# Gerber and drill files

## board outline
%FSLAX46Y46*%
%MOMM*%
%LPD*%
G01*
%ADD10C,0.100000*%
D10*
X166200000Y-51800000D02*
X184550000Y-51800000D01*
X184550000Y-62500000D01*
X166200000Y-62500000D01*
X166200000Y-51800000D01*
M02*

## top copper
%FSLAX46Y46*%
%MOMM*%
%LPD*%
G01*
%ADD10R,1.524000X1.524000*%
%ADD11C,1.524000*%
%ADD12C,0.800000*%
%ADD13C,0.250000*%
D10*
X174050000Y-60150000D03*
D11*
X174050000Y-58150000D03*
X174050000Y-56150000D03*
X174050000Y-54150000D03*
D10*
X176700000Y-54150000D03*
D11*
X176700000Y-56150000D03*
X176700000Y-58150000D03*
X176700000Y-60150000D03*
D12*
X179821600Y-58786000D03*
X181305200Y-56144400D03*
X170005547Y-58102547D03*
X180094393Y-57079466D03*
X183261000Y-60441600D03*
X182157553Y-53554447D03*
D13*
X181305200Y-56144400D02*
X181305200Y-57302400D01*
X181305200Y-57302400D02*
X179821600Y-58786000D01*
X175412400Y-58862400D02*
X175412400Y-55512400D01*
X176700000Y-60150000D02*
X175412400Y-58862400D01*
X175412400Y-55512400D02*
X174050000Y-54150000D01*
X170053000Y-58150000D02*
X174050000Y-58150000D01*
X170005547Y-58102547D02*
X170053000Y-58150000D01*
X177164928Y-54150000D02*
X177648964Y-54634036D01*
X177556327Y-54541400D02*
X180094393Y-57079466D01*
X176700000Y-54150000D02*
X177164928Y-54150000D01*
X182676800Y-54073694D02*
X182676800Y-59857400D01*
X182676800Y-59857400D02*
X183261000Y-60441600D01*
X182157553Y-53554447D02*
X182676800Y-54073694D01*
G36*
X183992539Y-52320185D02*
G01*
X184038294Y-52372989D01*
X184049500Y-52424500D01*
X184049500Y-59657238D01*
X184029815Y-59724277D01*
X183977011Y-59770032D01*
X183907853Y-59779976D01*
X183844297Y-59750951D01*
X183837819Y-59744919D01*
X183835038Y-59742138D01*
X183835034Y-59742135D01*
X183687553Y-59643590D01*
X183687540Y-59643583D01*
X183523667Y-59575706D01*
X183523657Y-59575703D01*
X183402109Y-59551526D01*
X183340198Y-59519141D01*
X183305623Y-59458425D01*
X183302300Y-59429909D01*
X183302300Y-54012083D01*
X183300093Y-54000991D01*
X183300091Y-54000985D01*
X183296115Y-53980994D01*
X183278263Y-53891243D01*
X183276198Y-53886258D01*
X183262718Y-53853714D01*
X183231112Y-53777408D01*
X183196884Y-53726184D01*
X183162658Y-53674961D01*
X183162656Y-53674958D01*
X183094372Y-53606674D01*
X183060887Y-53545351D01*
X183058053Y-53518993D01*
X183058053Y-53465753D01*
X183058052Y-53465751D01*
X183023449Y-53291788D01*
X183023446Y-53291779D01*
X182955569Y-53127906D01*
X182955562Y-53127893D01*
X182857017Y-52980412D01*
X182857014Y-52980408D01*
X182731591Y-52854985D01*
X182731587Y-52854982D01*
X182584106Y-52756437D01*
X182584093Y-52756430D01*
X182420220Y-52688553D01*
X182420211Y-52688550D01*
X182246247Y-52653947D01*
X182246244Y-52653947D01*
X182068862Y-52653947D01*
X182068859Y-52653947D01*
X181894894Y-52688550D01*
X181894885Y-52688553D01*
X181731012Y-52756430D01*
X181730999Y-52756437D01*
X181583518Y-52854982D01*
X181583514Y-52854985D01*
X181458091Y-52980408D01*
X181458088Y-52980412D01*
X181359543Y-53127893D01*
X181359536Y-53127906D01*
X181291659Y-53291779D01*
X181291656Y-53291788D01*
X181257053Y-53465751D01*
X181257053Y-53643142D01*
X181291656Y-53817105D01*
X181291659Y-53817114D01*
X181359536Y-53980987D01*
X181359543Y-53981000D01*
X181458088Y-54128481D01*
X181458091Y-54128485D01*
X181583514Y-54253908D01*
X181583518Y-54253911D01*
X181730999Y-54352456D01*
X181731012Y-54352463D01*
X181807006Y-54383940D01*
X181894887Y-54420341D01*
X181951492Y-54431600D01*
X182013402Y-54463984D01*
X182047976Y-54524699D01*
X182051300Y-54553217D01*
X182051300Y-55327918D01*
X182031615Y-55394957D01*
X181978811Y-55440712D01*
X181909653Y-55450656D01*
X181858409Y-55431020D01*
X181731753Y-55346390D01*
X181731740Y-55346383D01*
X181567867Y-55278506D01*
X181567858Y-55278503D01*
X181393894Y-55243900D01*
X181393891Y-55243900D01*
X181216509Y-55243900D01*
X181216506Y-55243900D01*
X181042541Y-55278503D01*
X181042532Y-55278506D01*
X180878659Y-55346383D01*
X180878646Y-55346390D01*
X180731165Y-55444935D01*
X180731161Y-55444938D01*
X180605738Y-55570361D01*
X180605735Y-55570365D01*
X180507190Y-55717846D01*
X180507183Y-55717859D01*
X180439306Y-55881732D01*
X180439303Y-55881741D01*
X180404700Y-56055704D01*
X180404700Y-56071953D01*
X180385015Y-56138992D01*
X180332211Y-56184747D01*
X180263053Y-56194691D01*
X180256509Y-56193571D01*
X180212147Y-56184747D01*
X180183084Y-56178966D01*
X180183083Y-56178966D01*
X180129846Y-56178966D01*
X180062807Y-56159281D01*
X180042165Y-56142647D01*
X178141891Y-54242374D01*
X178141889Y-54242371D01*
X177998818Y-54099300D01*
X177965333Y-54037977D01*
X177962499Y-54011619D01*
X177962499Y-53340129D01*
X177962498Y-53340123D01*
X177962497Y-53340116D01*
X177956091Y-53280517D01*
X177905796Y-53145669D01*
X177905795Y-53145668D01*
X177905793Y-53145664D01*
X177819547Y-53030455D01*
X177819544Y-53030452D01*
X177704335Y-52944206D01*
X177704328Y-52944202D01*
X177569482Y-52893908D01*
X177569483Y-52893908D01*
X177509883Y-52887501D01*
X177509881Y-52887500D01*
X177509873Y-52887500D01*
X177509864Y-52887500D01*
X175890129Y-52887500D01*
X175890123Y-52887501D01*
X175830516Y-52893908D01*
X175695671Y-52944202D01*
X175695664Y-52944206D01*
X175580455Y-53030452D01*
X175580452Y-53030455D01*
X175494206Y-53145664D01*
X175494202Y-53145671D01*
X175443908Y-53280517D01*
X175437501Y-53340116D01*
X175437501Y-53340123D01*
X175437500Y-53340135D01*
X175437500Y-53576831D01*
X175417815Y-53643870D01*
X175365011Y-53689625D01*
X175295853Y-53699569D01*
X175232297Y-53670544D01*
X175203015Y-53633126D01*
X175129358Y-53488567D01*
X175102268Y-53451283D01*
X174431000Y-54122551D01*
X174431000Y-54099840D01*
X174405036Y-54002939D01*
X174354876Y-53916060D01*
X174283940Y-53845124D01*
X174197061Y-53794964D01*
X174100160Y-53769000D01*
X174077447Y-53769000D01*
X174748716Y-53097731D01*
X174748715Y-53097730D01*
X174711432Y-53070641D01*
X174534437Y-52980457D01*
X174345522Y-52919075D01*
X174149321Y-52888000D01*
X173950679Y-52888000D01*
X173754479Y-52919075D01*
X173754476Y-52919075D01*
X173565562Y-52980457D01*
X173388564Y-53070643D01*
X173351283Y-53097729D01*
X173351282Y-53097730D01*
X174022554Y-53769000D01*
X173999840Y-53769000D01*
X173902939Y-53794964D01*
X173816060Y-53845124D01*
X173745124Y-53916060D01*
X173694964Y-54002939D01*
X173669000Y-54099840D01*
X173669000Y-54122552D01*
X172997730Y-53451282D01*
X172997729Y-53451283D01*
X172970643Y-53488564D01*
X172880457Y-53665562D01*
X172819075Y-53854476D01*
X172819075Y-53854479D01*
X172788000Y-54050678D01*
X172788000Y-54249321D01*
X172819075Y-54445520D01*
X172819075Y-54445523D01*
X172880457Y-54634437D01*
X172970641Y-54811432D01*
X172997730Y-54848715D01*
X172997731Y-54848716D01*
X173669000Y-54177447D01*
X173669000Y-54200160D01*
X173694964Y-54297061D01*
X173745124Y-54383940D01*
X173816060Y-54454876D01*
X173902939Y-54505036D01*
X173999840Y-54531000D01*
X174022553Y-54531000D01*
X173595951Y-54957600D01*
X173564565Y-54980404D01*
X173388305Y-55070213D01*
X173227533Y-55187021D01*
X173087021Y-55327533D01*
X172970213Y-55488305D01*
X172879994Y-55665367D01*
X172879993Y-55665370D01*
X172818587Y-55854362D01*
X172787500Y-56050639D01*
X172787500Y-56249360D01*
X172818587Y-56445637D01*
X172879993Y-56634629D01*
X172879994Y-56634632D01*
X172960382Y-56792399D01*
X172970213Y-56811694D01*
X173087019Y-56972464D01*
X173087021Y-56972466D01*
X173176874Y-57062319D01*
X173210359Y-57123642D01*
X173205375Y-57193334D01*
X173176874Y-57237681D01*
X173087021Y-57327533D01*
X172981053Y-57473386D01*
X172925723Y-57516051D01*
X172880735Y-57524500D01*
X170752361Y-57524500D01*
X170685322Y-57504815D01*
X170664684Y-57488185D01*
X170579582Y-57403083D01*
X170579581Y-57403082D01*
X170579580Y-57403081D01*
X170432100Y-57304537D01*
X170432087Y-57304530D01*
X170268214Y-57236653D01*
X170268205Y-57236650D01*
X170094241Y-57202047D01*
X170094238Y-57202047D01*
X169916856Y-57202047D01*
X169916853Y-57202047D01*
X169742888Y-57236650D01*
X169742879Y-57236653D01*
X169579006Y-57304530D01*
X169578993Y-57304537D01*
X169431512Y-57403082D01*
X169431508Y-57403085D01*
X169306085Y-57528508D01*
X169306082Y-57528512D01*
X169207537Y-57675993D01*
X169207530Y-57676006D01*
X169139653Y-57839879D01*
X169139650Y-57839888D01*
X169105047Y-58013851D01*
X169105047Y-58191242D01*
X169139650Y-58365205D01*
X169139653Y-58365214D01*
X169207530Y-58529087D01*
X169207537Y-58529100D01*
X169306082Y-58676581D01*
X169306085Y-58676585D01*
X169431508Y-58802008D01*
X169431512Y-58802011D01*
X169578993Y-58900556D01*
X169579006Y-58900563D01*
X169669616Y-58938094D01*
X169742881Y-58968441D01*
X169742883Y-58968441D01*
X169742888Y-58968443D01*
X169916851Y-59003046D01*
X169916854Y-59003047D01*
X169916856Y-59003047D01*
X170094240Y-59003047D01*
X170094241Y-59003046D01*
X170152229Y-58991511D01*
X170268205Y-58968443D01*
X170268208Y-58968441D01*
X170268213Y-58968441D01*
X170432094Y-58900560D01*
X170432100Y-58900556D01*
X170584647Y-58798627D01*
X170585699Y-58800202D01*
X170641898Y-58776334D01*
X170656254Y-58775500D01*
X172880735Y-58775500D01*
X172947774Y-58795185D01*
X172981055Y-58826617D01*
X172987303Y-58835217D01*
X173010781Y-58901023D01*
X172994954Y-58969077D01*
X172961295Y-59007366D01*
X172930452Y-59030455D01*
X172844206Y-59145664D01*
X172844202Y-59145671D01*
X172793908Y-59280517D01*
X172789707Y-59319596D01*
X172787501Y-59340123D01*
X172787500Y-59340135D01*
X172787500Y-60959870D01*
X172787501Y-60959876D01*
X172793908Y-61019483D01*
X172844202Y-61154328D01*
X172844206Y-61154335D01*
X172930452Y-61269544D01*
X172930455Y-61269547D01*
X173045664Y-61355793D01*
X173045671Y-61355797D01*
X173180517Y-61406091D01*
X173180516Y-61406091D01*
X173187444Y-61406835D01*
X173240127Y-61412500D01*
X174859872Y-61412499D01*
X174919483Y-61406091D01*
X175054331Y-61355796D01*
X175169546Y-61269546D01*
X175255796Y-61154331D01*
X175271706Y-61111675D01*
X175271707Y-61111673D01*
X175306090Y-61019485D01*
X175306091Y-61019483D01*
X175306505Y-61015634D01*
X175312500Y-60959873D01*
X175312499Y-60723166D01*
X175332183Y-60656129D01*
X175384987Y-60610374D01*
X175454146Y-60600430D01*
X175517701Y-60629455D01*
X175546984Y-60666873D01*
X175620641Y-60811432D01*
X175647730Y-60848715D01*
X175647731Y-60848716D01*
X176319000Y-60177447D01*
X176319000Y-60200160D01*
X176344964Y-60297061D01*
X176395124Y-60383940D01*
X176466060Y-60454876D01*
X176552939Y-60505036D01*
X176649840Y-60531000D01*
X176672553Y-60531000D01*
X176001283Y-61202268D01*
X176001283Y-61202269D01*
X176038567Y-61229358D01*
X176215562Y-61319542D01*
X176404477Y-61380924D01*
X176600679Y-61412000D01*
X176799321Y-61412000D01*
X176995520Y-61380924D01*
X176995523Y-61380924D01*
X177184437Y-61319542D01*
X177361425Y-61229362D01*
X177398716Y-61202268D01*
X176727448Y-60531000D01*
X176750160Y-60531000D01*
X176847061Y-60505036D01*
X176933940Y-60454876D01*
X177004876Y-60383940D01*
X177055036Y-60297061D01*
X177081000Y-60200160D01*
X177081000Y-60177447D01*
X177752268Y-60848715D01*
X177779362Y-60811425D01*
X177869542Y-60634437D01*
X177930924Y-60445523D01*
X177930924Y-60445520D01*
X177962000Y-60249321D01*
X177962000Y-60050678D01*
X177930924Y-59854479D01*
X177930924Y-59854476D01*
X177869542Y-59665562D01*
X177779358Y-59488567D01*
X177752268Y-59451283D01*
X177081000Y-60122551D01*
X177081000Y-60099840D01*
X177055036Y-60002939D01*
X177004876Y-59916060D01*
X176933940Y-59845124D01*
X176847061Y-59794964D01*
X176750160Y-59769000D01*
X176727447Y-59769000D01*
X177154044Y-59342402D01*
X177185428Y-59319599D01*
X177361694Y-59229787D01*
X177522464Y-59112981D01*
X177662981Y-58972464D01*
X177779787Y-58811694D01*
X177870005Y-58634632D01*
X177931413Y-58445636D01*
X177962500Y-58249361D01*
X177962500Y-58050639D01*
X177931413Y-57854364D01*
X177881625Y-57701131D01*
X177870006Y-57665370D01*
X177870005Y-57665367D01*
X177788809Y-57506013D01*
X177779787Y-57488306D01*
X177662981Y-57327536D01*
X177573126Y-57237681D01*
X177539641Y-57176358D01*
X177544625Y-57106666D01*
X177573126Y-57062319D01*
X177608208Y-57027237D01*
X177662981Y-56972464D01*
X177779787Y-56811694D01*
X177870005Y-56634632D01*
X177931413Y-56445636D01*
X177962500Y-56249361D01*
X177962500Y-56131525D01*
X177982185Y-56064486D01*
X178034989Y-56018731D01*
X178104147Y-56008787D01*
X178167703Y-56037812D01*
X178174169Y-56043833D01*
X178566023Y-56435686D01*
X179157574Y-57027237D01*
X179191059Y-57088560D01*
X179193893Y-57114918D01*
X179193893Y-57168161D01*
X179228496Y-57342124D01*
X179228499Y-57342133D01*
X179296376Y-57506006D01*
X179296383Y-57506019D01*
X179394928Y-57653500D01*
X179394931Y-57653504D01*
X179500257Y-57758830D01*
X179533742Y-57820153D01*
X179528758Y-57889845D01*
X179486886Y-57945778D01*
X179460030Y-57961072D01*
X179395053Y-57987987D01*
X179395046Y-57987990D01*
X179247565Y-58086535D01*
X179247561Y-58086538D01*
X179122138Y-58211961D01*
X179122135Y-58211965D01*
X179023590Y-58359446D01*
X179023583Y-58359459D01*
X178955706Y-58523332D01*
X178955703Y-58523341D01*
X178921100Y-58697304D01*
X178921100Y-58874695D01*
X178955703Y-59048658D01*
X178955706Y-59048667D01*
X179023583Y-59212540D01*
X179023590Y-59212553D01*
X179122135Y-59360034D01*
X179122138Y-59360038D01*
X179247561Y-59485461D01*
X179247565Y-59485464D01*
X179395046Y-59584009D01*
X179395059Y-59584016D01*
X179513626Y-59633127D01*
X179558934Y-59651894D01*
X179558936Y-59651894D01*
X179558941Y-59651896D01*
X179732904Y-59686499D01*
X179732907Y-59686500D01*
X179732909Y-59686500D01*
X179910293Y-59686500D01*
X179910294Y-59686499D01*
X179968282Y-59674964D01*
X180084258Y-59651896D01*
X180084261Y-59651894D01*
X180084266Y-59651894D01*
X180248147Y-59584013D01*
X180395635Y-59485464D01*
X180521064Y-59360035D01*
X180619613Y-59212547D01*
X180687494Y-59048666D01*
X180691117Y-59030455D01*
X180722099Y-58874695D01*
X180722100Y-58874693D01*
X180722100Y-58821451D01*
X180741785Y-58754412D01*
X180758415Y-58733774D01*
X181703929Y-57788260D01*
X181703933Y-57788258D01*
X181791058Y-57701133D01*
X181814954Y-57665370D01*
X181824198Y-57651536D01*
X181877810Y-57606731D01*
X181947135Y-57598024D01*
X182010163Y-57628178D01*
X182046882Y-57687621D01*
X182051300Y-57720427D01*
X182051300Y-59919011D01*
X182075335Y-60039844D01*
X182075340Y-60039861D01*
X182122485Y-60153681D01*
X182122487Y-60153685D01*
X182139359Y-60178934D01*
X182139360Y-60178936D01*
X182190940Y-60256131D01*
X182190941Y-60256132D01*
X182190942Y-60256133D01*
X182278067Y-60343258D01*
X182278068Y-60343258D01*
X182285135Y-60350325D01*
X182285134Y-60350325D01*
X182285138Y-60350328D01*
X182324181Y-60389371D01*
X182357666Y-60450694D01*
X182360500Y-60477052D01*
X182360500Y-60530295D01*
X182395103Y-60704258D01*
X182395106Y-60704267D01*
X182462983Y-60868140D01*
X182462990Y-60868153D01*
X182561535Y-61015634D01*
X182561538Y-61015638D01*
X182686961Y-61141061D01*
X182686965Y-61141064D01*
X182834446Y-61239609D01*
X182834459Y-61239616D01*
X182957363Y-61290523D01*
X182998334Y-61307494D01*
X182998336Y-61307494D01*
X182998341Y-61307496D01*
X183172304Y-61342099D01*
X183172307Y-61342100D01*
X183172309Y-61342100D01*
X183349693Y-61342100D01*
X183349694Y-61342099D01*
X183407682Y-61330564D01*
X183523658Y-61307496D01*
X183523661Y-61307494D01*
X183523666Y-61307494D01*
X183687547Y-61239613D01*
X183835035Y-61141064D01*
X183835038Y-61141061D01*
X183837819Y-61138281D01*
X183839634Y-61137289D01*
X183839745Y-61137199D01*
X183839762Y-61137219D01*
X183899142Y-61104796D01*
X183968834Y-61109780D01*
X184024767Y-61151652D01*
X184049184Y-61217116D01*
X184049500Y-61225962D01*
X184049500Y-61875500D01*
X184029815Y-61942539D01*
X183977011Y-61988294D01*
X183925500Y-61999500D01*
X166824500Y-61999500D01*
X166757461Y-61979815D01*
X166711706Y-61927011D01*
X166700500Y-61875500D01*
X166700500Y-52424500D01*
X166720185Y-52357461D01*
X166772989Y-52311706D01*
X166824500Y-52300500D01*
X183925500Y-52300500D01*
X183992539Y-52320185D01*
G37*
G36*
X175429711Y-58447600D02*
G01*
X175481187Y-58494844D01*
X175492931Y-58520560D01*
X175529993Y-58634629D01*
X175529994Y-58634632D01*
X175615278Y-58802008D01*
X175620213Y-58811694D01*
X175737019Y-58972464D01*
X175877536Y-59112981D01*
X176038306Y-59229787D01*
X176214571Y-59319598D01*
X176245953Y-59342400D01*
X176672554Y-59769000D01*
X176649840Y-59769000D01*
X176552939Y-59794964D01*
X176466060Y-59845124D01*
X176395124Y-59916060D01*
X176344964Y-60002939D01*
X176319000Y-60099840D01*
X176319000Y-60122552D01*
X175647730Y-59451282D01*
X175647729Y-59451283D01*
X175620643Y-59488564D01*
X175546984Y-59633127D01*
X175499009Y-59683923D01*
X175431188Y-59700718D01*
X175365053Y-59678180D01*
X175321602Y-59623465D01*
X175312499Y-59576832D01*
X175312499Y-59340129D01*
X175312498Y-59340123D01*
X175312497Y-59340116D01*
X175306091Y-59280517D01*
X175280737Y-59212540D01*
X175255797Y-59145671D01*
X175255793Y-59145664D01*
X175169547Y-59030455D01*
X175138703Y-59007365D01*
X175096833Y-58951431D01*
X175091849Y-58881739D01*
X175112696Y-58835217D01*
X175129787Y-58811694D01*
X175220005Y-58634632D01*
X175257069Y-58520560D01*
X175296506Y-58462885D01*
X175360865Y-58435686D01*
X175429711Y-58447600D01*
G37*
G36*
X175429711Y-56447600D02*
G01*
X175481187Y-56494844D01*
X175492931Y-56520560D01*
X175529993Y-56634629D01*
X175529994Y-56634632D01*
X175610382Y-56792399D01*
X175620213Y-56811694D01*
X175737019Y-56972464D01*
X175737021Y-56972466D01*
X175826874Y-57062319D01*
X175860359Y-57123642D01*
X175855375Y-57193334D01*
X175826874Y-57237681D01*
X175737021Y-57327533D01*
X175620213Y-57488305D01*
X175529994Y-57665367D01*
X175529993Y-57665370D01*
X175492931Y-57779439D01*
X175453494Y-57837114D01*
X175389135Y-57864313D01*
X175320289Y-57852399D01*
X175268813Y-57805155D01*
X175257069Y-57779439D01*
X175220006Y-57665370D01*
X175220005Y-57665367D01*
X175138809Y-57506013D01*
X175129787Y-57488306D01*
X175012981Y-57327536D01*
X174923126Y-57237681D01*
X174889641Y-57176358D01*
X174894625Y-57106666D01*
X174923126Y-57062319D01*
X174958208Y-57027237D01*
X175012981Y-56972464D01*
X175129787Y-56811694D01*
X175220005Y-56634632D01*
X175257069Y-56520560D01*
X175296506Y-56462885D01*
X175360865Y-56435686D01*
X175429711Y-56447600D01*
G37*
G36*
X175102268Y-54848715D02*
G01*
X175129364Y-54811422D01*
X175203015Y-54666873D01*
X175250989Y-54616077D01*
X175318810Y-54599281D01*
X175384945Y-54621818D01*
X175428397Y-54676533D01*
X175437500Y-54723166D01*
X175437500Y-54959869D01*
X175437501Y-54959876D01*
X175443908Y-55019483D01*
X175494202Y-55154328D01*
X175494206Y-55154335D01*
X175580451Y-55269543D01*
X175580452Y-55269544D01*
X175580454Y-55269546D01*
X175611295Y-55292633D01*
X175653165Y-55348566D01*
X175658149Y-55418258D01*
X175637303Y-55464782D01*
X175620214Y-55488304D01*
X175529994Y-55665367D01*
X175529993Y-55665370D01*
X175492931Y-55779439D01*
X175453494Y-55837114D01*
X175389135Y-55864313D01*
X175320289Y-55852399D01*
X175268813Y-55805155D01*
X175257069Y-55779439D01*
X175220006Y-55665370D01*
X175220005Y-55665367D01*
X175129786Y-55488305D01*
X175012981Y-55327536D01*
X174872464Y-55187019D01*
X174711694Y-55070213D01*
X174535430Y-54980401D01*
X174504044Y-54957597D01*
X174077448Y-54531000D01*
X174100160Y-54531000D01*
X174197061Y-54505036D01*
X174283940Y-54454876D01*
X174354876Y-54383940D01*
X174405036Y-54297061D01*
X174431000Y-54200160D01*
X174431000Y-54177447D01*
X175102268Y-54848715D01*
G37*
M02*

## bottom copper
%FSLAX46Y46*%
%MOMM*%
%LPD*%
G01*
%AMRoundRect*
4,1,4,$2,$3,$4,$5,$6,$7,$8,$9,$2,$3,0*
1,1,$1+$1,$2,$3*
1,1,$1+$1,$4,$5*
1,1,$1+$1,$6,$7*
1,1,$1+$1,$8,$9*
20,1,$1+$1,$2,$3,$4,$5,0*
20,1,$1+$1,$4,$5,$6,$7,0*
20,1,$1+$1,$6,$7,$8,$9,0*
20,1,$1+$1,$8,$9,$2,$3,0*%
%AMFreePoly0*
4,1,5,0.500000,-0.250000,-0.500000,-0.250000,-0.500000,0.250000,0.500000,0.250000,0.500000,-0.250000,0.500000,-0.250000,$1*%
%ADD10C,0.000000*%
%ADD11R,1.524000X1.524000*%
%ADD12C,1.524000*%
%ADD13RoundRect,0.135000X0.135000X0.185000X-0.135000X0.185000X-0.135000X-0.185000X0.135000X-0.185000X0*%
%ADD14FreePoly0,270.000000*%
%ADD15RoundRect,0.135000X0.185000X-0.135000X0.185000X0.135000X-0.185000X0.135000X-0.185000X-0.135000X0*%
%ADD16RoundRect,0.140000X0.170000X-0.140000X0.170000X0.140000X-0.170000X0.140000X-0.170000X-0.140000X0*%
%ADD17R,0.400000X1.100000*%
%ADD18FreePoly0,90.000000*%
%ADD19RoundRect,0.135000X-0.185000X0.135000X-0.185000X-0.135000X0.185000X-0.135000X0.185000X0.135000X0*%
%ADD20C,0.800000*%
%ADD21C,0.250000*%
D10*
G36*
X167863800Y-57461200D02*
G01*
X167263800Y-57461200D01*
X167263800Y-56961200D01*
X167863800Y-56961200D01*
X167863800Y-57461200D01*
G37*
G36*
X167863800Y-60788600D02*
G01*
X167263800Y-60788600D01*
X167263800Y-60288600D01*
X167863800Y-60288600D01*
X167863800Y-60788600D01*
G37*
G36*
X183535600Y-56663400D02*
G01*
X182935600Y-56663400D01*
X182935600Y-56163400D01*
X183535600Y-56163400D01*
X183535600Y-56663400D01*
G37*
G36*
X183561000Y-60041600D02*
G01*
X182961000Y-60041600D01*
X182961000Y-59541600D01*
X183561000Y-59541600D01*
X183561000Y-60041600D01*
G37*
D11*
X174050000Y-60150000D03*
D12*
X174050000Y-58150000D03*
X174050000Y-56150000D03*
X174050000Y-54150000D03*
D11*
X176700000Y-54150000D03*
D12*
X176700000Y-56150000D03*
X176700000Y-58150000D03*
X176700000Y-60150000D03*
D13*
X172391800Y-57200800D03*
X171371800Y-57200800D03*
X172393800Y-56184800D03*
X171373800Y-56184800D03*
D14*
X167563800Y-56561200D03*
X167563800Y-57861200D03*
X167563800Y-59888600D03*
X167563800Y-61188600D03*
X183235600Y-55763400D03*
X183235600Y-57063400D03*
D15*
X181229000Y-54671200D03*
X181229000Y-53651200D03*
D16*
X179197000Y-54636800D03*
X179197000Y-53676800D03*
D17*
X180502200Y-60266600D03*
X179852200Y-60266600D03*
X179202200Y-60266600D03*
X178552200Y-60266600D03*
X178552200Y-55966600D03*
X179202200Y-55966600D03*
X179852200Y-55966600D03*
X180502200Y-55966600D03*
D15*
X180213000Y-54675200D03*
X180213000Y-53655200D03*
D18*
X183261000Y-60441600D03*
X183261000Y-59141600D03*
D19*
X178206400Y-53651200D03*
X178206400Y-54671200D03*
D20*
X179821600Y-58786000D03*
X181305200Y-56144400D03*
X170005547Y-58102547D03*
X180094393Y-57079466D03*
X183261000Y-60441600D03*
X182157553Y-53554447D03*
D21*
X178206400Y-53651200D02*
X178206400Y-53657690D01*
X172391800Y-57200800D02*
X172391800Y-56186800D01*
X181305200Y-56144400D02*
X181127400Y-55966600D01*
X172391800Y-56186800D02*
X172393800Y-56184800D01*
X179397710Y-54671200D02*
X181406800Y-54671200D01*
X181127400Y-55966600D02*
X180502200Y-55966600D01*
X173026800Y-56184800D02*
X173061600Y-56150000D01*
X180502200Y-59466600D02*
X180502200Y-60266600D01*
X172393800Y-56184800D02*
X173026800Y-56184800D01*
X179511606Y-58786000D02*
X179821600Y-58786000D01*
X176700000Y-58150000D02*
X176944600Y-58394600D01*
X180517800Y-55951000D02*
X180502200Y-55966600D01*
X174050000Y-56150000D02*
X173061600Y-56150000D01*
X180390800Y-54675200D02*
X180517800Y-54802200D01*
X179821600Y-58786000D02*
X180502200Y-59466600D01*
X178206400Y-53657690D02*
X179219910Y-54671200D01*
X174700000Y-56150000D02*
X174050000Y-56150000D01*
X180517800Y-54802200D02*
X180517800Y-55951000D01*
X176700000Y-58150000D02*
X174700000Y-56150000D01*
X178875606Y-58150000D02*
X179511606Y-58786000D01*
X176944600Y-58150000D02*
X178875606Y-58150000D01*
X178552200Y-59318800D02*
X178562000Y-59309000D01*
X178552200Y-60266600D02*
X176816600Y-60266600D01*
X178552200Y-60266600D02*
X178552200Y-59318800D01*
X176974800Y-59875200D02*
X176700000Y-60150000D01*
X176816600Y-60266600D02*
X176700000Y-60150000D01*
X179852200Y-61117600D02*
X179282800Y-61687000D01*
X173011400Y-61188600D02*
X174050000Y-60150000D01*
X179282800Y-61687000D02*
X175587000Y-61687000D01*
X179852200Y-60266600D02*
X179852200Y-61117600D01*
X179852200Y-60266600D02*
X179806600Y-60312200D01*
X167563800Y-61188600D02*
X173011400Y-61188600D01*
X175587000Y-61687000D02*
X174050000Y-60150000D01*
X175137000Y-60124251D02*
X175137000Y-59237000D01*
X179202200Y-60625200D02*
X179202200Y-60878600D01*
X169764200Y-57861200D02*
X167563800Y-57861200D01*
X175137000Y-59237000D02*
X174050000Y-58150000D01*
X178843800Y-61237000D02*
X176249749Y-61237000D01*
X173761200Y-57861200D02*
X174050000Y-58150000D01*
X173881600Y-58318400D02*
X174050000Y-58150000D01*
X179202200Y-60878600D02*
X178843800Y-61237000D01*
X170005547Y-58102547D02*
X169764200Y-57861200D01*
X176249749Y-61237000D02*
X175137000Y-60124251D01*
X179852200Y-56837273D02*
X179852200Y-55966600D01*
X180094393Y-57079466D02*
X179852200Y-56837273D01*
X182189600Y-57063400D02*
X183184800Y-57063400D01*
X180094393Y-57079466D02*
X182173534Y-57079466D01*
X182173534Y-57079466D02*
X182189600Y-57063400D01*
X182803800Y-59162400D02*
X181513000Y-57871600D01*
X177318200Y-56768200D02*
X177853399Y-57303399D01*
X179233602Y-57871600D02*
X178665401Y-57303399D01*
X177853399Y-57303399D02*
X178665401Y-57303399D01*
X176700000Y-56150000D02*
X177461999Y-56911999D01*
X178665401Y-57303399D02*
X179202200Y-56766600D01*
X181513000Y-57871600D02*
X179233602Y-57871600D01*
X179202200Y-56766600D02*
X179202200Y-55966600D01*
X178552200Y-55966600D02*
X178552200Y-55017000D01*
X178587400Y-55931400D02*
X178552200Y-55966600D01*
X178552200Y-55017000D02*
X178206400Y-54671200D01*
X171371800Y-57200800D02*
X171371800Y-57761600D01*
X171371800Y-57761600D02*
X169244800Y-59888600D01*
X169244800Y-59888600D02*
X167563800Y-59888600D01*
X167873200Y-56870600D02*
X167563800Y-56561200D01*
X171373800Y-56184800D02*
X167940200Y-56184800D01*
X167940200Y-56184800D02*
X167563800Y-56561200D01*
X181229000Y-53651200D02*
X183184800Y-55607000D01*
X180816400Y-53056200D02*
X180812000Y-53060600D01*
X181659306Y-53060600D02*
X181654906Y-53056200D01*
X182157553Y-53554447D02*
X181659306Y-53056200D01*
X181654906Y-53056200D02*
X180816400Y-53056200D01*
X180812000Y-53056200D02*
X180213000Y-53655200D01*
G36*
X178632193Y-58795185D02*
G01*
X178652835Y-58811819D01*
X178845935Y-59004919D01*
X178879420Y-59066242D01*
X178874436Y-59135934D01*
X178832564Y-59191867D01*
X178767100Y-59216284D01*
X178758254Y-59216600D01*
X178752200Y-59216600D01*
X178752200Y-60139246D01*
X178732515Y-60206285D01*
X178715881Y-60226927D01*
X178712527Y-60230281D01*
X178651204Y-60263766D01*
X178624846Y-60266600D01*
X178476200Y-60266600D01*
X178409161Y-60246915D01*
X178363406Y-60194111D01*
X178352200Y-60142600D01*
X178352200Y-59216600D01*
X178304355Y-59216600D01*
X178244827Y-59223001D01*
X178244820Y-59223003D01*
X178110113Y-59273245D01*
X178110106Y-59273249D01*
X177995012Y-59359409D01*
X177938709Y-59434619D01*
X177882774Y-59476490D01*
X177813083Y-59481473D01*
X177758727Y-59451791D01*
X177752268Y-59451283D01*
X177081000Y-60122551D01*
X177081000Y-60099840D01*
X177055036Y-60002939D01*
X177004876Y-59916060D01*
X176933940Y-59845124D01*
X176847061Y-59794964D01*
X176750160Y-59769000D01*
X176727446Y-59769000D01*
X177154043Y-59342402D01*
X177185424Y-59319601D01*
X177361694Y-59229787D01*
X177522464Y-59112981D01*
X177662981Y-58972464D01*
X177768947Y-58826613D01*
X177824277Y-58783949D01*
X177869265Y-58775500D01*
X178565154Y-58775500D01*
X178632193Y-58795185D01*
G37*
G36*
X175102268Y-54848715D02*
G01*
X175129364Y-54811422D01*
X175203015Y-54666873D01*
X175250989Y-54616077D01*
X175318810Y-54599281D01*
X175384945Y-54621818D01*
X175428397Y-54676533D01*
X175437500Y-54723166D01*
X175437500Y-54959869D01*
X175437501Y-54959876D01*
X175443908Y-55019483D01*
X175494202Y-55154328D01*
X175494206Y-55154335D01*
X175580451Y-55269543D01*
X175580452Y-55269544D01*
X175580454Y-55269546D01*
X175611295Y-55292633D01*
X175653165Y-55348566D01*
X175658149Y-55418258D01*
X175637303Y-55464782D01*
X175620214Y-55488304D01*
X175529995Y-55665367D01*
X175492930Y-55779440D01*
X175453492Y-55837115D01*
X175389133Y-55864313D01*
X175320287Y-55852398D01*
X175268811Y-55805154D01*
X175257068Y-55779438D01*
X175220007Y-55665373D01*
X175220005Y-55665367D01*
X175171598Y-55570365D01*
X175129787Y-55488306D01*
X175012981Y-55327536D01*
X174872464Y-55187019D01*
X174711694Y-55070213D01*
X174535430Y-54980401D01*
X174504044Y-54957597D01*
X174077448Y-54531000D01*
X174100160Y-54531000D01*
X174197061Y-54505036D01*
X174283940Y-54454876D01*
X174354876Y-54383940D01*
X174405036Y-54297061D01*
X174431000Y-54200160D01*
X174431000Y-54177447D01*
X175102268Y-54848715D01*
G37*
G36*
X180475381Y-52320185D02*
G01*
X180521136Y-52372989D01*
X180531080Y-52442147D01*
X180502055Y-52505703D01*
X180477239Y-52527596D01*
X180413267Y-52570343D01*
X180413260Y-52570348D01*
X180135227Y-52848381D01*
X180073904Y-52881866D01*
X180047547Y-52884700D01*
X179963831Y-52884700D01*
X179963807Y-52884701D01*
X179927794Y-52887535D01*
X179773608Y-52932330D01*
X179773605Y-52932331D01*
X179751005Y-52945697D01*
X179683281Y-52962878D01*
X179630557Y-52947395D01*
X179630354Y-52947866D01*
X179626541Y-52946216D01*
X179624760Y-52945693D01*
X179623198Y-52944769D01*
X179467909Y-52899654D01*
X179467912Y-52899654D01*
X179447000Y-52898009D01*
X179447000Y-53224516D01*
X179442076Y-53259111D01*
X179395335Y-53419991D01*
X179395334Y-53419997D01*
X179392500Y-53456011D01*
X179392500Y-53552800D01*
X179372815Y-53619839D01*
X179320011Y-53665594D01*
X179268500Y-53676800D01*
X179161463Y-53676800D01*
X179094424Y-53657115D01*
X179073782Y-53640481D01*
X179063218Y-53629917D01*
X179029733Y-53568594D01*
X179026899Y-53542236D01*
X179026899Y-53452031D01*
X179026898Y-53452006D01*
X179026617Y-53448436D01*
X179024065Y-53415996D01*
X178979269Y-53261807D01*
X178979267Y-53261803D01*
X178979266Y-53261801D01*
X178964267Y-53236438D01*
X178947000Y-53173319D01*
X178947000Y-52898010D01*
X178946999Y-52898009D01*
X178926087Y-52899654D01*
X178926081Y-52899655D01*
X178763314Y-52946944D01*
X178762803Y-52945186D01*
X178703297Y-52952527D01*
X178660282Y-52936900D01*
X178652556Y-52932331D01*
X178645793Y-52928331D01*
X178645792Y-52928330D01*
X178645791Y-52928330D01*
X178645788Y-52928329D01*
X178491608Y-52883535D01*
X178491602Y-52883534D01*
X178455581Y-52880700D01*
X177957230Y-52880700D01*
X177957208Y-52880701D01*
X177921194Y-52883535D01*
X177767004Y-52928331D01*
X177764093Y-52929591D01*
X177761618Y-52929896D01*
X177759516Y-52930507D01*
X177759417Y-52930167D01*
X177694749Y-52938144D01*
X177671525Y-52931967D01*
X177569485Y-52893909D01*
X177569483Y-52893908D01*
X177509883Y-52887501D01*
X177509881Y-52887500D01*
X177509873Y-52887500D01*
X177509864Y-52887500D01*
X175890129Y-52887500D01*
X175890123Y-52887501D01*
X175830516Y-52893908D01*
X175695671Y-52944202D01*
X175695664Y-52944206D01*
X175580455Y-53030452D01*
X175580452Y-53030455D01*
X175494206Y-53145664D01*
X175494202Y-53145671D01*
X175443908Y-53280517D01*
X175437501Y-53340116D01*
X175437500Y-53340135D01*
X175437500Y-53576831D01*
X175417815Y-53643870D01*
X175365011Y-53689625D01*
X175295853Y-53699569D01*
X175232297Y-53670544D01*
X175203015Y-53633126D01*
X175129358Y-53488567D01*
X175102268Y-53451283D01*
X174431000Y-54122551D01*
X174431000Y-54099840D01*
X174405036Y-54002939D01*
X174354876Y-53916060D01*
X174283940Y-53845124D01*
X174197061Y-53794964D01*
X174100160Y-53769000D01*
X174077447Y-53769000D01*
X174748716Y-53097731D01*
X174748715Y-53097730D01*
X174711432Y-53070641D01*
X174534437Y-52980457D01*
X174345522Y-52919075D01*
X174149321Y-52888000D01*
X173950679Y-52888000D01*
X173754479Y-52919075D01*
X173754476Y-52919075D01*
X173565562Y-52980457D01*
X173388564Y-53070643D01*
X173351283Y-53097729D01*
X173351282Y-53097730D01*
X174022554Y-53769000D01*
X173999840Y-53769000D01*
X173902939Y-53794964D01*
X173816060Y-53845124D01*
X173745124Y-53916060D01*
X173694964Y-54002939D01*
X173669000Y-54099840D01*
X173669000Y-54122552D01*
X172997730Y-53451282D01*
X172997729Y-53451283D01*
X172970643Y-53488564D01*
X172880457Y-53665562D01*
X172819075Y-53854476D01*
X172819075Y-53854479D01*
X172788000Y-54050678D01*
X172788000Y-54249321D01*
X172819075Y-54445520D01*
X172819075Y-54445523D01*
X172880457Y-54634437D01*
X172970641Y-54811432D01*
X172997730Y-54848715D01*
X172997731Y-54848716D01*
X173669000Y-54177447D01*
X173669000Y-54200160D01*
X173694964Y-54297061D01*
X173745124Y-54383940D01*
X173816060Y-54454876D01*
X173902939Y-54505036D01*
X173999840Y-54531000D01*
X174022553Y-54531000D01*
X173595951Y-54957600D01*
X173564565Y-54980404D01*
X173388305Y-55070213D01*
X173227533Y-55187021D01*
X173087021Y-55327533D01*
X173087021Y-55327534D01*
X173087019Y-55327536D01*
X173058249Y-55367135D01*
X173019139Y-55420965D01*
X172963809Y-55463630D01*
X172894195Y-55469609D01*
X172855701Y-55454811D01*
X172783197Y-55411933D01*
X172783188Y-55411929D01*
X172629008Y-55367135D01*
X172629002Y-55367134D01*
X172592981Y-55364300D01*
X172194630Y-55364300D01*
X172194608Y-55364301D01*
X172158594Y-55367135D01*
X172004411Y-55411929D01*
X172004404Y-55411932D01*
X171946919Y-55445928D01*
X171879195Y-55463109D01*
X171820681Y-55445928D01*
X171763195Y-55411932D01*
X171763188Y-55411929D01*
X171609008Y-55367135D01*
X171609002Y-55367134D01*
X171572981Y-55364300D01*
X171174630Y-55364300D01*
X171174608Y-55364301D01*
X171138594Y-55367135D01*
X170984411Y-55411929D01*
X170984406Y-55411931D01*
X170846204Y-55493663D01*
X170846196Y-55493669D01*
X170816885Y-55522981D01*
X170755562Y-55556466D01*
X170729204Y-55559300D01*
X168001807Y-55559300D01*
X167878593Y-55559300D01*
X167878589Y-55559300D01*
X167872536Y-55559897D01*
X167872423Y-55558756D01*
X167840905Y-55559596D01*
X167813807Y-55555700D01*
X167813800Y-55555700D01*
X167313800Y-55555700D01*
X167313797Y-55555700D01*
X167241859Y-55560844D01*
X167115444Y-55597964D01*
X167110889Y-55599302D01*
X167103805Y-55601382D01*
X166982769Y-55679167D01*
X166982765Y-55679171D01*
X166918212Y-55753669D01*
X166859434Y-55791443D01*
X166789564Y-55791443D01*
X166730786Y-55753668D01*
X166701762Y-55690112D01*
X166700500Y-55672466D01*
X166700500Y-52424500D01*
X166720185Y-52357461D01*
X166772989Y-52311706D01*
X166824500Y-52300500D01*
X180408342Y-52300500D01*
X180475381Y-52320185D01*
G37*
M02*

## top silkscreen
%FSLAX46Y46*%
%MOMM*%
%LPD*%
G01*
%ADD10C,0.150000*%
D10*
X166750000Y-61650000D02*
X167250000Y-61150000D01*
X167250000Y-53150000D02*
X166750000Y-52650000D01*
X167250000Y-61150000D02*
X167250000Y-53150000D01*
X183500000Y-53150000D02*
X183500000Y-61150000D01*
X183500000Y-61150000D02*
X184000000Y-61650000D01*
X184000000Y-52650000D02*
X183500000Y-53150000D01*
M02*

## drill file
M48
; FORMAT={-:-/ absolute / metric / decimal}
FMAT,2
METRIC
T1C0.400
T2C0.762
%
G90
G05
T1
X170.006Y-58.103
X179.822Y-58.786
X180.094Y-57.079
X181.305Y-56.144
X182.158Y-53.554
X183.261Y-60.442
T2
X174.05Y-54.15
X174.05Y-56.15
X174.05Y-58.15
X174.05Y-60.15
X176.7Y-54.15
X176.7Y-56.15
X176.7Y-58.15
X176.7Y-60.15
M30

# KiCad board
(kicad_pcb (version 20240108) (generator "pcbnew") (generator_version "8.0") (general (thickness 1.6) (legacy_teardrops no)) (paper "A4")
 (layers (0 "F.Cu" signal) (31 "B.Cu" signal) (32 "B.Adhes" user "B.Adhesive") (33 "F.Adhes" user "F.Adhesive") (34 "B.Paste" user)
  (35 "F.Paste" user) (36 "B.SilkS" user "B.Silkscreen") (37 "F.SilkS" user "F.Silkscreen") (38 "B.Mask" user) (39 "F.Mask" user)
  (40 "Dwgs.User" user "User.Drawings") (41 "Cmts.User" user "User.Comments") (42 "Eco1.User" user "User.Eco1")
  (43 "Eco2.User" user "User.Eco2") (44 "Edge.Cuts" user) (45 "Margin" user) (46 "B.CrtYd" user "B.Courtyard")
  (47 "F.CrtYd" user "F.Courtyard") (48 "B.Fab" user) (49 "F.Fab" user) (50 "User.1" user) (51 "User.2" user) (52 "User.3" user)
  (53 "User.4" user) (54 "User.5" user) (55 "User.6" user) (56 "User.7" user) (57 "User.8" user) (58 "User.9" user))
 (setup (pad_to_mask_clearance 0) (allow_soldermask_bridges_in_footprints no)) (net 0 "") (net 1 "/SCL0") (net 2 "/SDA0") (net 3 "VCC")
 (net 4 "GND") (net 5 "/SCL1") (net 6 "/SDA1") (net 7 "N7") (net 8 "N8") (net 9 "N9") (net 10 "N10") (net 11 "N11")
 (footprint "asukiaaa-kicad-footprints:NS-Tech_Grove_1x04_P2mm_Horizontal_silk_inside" (layer "F.Cu") (at 174.05 57.15 180)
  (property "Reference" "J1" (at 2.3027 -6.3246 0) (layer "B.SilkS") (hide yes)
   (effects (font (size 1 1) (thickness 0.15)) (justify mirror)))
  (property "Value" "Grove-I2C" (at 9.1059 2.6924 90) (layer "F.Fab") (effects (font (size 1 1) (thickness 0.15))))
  (fp_line (start 7.3 -4.5) (end 6.8 -4) (stroke (width 0.15) (type solid)) (layer "F.SilkS"))
  (fp_line (start 6.8 4) (end 7.3 4.5) (stroke (width 0.15) (type solid)) (layer "F.SilkS"))
  (fp_line (start 6.8 -4) (end 6.8 4) (stroke (width 0.15) (type solid)) (layer "F.SilkS"))
  (pad "1" thru_hole rect (at 0 -3 180) (size 1.524 1.524) (drill 0.762) (layers "*.Cu" "*.Mask") (remove_unused_layers no) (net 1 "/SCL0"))
  (pad "2" thru_hole circle (at 0 -1 180) (size 1.524 1.524) (drill 0.762) (layers "*.Cu" "*.Mask") (remove_unused_layers no)
   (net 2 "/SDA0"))
  (pad "3" thru_hole circle (at 0 1 180) (size 1.524 1.524) (drill 0.762) (layers "*.Cu" "*.Mask") (remove_unused_layers no) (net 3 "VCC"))
  (pad "4" thru_hole circle (at 0 3 180) (size 1.524 1.524) (drill 0.762) (layers "*.Cu" "*.Mask") (remove_unused_layers no) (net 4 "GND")))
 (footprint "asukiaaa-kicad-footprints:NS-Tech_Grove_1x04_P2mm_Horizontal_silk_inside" (layer "F.Cu") (at 176.7 57.15)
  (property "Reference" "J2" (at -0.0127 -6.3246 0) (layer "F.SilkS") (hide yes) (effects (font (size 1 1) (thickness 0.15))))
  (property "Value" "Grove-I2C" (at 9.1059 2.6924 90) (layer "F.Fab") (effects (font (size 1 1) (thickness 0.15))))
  (fp_line (start 6.8 -4) (end 6.8 4) (stroke (width 0.15) (type solid)) (layer "F.SilkS"))
  (fp_line (start 6.8 4) (end 7.3 4.5) (stroke (width 0.15) (type solid)) (layer "F.SilkS"))
  (fp_line (start 7.3 -4.5) (end 6.8 -4) (stroke (width 0.15) (type solid)) (layer "F.SilkS"))
  (pad "1" thru_hole rect (at 0 -3) (size 1.524 1.524) (drill 0.762) (layers "*.Cu" "*.Mask") (remove_unused_layers no) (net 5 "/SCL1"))
  (pad "2" thru_hole circle (at 0 -1) (size 1.524 1.524) (drill 0.762) (layers "*.Cu" "*.Mask") (remove_unused_layers no) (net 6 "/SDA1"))
  (pad "3" thru_hole circle (at 0 1) (size 1.524 1.524) (drill 0.762) (layers "*.Cu" "*.Mask") (remove_unused_layers no) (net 3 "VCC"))
  (pad "4" thru_hole circle (at 0 3) (size 1.524 1.524) (drill 0.762) (layers "*.Cu" "*.Mask") (remove_unused_layers no) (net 4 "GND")))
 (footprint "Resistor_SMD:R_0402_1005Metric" (layer "B.Cu") (at 171.8818 57.2008 180)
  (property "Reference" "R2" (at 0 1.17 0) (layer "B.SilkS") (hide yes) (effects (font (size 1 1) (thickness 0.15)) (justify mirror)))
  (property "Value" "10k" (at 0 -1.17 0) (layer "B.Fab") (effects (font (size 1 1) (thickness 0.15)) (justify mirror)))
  (pad "1" smd roundrect (at -0.51 0 180) (size 0.54 0.64) (layers "B.Cu" "B.Paste" "B.Mask") (roundrect_rratio 0.25) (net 3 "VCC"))
  (pad "2" smd roundrect (at 0.51 0 180) (size 0.54 0.64) (layers "B.Cu" "B.Paste" "B.Mask") (roundrect_rratio 0.25) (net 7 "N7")))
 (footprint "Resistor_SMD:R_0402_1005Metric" (layer "B.Cu") (at 171.8838 56.1848 180)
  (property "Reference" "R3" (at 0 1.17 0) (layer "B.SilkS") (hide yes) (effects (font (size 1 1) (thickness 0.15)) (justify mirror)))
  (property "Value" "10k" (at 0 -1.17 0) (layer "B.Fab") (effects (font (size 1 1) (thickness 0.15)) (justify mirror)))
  (pad "1" smd roundrect (at -0.51 0 180) (size 0.54 0.64) (layers "B.Cu" "B.Paste" "B.Mask") (roundrect_rratio 0.25) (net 3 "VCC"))
  (pad "2" smd roundrect (at 0.51 0 180) (size 0.54 0.64) (layers "B.Cu" "B.Paste" "B.Mask") (roundrect_rratio 0.25) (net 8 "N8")))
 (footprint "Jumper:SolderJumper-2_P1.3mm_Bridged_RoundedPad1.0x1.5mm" (layer "B.Cu") (at 167.5638 57.2112 -90)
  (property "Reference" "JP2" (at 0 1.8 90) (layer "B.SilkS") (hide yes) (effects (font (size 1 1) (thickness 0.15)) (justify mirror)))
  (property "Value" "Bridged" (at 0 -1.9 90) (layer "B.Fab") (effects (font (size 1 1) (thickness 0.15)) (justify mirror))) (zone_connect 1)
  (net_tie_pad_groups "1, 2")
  (fp_poly (pts (xy 0.25 0.3) (xy -0.25 0.3) (xy -0.25 -0.3) (xy 0.25 -0.3)) (stroke (width 0) (type solid)) (fill solid) (layer "B.Cu"))
  (pad "1" smd custom (at -0.65 0 270) (size 1 0.5) (layers "B.Cu" "B.Mask") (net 8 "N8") (zone_connect 2) (thermal_bridge_angle 45)
   (options (clearance outline) (anchor rect)) (primitives))
  (pad "2" smd custom (at 0.65 0 270) (size 1 0.5) (layers "B.Cu" "B.Mask") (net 2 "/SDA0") (zone_connect 2) (thermal_bridge_angle 45)
   (options (clearance outline) (anchor rect)) (primitives)))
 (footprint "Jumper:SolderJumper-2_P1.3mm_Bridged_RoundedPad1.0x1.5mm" (layer "B.Cu") (at 167.5638 60.5386 -90)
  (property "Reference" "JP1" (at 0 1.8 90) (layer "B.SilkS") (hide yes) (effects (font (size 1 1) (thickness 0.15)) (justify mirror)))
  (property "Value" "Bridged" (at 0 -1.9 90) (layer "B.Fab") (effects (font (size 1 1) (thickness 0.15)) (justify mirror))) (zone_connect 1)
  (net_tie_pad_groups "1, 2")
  (fp_poly (pts (xy 0.25 0.3) (xy -0.25 0.3) (xy -0.25 -0.3) (xy 0.25 -0.3)) (stroke (width 0) (type solid)) (fill solid) (layer "B.Cu"))
  (pad "1" smd custom (at -0.65 0 270) (size 1 0.5) (layers "B.Cu" "B.Mask") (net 7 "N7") (zone_connect 2) (thermal_bridge_angle 45)
   (options (clearance outline) (anchor rect)) (primitives))
  (pad "2" smd custom (at 0.65 0 270) (size 1 0.5) (layers "B.Cu" "B.Mask") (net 1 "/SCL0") (zone_connect 2) (thermal_bridge_angle 45)
   (options (clearance outline) (anchor rect)) (primitives)))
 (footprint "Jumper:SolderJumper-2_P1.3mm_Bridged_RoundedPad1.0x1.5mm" (layer "B.Cu") (at 183.2356 56.4134 -90)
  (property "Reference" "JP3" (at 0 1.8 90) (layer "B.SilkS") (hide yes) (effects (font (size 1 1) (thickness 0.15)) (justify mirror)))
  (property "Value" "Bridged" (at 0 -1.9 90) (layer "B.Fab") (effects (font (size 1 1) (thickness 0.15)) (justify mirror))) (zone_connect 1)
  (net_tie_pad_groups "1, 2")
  (fp_poly (pts (xy 0.25 0.3) (xy -0.25 0.3) (xy -0.25 -0.3) (xy 0.25 -0.3)) (stroke (width 0) (type solid)) (fill solid) (layer "B.Cu"))
  (pad "1" smd custom (at -0.65 0 270) (size 1 0.5) (layers "B.Cu" "B.Mask") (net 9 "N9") (zone_connect 2) (thermal_bridge_angle 45)
   (options (clearance outline) (anchor rect)) (primitives))
  (pad "2" smd custom (at 0.65 0 270) (size 1 0.5) (layers "B.Cu" "B.Mask") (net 5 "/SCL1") (zone_connect 2) (thermal_bridge_angle 45)
   (options (clearance outline) (anchor rect)) (primitives)))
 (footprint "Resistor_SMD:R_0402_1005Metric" (layer "B.Cu") (at 181.229 54.1612 90)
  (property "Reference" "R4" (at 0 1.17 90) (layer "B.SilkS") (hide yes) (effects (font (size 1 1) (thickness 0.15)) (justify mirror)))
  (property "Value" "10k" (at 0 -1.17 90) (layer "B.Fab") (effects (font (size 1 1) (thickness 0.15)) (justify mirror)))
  (pad "1" smd roundrect (at -0.51 0 90) (size 0.54 0.64) (layers "B.Cu" "B.Paste" "B.Mask") (roundrect_rratio 0.25) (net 3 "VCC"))
  (pad "2" smd roundrect (at 0.51 0 90) (size 0.54 0.64) (layers "B.Cu" "B.Paste" "B.Mask") (roundrect_rratio 0.25) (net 9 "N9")))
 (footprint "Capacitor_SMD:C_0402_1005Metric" (layer "B.Cu") (at 179.197 54.1568 90)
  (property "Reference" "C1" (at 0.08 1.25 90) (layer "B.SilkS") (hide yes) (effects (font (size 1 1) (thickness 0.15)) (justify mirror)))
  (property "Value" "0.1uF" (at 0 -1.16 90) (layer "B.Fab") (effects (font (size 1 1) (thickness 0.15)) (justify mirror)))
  (pad "1" smd roundrect (at -0.48 0 90) (size 0.56 0.62) (layers "B.Cu" "B.Paste" "B.Mask") (roundrect_rratio 0.25) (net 3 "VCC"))
  (pad "2" smd roundrect (at 0.48 0 90) (size 0.56 0.62) (layers "B.Cu" "B.Paste" "B.Mask") (roundrect_rratio 0.25) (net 4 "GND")))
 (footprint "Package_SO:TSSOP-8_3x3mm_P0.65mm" (layer "B.Cu") (at 179.5272 58.1166 90)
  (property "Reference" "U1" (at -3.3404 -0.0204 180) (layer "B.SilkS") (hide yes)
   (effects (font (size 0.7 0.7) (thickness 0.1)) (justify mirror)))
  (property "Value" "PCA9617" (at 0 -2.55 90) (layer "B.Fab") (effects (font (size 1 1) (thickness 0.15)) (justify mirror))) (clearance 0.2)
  (pad "1" smd rect (at -2.15 0.975 90) (size 1.1 0.4) (layers "B.Cu" "B.Paste" "B.Mask") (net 3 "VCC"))
  (pad "2" smd rect (at -2.15 0.325 90) (size 1.1 0.4) (layers "B.Cu" "B.Paste" "B.Mask") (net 1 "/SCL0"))
  (pad "3" smd rect (at -2.15 -0.325 90) (size 1.1 0.4) (layers "B.Cu" "B.Paste" "B.Mask") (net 2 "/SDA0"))
  (pad "4" smd rect (at -2.15 -0.975 90) (size 1.1 0.4) (layers "B.Cu" "B.Paste" "B.Mask") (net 4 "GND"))
  (pad "5" smd rect (at 2.15 -0.975 90) (size 1.1 0.4) (layers "B.Cu" "B.Paste" "B.Mask") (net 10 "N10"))
  (pad "6" smd rect (at 2.15 -0.325 90) (size 1.1 0.4) (layers "B.Cu" "B.Paste" "B.Mask") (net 6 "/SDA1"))
  (pad "7" smd rect (at 2.15 0.325 90) (size 1.1 0.4) (layers "B.Cu" "B.Paste" "B.Mask") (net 5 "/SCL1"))
  (pad "8" smd rect (at 2.15 0.975 90) (size 1.1 0.4) (layers "B.Cu" "B.Paste" "B.Mask") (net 3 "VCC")))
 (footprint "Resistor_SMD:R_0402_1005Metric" (layer "B.Cu") (at 180.213 54.1652 90)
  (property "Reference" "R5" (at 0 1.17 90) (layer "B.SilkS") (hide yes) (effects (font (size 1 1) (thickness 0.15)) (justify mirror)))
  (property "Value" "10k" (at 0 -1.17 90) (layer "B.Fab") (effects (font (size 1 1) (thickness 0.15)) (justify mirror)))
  (pad "1" smd roundrect (at -0.51 0 90) (size 0.54 0.64) (layers "B.Cu" "B.Paste" "B.Mask") (roundrect_rratio 0.25) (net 3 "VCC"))
  (pad "2" smd roundrect (at 0.51 0 90) (size 0.54 0.64) (layers "B.Cu" "B.Paste" "B.Mask") (roundrect_rratio 0.25) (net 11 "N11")))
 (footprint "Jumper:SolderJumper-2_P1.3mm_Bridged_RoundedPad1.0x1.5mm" (layer "B.Cu") (at 183.261 59.7916 90)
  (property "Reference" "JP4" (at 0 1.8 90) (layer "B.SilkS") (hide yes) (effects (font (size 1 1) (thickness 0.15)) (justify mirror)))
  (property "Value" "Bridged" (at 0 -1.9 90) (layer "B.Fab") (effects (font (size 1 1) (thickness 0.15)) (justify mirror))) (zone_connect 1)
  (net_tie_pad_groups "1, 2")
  (fp_poly (pts (xy 0.25 0.3) (xy -0.25 0.3) (xy -0.25 -0.3) (xy 0.25 -0.3)) (stroke (width 0) (type solid)) (fill solid) (layer "B.Cu"))
  (pad "1" smd custom (at -0.65 0 90) (size 1 0.5) (layers "B.Cu" "B.Mask") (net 11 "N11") (zone_connect 2) (thermal_bridge_angle 45)
   (options (clearance outline) (anchor rect)) (primitives))
  (pad "2" smd custom (at 0.65 0 90) (size 1 0.5) (layers "B.Cu" "B.Mask") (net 6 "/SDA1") (zone_connect 2) (thermal_bridge_angle 45)
   (options (clearance outline) (anchor rect)) (primitives)))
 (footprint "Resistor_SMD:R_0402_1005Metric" (layer "B.Cu") (at 178.2064 54.1612 -90)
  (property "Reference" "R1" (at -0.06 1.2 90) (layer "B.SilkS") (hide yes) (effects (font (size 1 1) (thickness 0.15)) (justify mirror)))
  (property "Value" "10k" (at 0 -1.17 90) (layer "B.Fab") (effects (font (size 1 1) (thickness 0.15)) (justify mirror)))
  (pad "1" smd roundrect (at -0.51 0 270) (size 0.54 0.64) (layers "B.Cu" "B.Paste" "B.Mask") (roundrect_rratio 0.25) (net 3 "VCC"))
  (pad "2" smd roundrect (at 0.51 0 270) (size 0.54 0.64) (layers "B.Cu" "B.Paste" "B.Mask") (roundrect_rratio 0.25) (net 10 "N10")))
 (gr_rect (start 166.2 51.8) (end 184.55 62.5) (stroke (width 0.1) (type default)) (fill none) (layer "Edge.Cuts"))
 (segment (start 181.3052 56.1444) (end 181.3052 57.3024) (width 0.25) (layer "F.Cu") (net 3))
 (segment (start 181.3052 57.3024) (end 179.8216 58.786) (width 0.25) (layer "F.Cu") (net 3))
 (via (at 179.8216 58.786) (size 0.8) (drill 0.4) (layers "F.Cu" "B.Cu") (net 3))
 (via (at 181.3052 56.1444) (size 0.8) (drill 0.4) (layers "F.Cu" "B.Cu") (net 3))
 (segment (start 178.2064 53.6512) (end 178.2064 53.65769) (width 0.25) (layer "B.Cu") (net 3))
 (segment (start 172.3918 57.2008) (end 172.3918 56.1868) (width 0.25) (layer "B.Cu") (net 3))
 (segment (start 181.3052 56.1444) (end 181.1274 55.9666) (width 0.25) (layer "B.Cu") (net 3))
 (segment (start 172.3918 56.1868) (end 172.3938 56.1848) (width 0.25) (layer "B.Cu") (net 3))
 (segment (start 179.39771 54.6712) (end 181.4068 54.6712) (width 0.25) (layer "B.Cu") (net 3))
 (segment (start 181.1274 55.9666) (end 180.5022 55.9666) (width 0.25) (layer "B.Cu") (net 3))
 (segment (start 173.0268 56.1848) (end 173.0616 56.15) (width 0.25) (layer "B.Cu") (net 3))
 (segment (start 180.5022 59.4666) (end 180.5022 60.2666) (width 0.25) (layer "B.Cu") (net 3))
 (segment (start 172.3938 56.1848) (end 173.0268 56.1848) (width 0.25) (layer "B.Cu") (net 3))
 (segment (start 179.511606 58.786) (end 179.8216 58.786) (width 0.25) (layer "B.Cu") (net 3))
 (segment (start 176.7 58.15) (end 176.9446 58.3946) (width 0.25) (layer "B.Cu") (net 3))
 (segment (start 180.5178 55.951) (end 180.5022 55.9666) (width 0.25) (layer "B.Cu") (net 3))
 (segment (start 174.05 56.15) (end 173.0616 56.15) (width 0.25) (layer "B.Cu") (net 3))
 (segment (start 180.3908 54.6752) (end 180.5178 54.8022) (width 0.25) (layer "B.Cu") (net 3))
 (segment (start 179.8216 58.786) (end 180.5022 59.4666) (width 0.25) (layer "B.Cu") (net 3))
 (segment (start 178.2064 53.65769) (end 179.21991 54.6712) (width 0.25) (layer "B.Cu") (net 3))
 (segment (start 174.7 56.15) (end 174.05 56.15) (width 0.25) (layer "B.Cu") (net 3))
 (segment (start 180.5178 54.8022) (end 180.5178 55.951) (width 0.25) (layer "B.Cu") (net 3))
 (segment (start 176.7 58.15) (end 174.7 56.15) (width 0.25) (layer "B.Cu") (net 3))
 (segment (start 178.875606 58.15) (end 179.511606 58.786) (width 0.25) (layer "B.Cu") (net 3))
 (segment (start 176.9446 58.15) (end 178.875606 58.15) (width 0.25) (layer "B.Cu") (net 3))
 (segment (start 175.4124 58.8624) (end 175.4124 55.5124) (width 0.25) (layer "F.Cu") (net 4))
 (segment (start 176.7 60.15) (end 175.4124 58.8624) (width 0.25) (layer "F.Cu") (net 4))
 (segment (start 175.4124 55.5124) (end 174.05 54.15) (width 0.25) (layer "F.Cu") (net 4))
 (segment (start 178.5522 59.3188) (end 178.562 59.309) (width 0.25) (layer "B.Cu") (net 4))
 (segment (start 178.5522 60.2666) (end 176.8166 60.2666) (width 0.25) (layer "B.Cu") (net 4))
 (segment (start 178.5522 60.2666) (end 178.5522 59.3188) (width 0.25) (layer "B.Cu") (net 4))
 (segment (start 176.9748 59.8752) (end 176.7 60.15) (width 0.25) (layer "B.Cu") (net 4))
 (segment (start 176.8166 60.2666) (end 176.7 60.15) (width 0.25) (layer "B.Cu") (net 4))
 (segment (start 179.8522 61.1176) (end 179.2828 61.687) (width 0.25) (layer "B.Cu") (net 1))
 (segment (start 173.0114 61.1886) (end 174.05 60.15) (width 0.25) (layer "B.Cu") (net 1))
 (segment (start 179.2828 61.687) (end 175.587 61.687) (width 0.25) (layer "B.Cu") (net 1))
 (segment (start 179.8522 60.2666) (end 179.8522 61.1176) (width 0.25) (layer "B.Cu") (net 1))
 (segment (start 179.8522 60.2666) (end 179.8066 60.3122) (width 0.25) (layer "B.Cu") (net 1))
 (segment (start 167.5638 61.1886) (end 173.0114 61.1886) (width 0.25) (layer "B.Cu") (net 1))
 (segment (start 175.587 61.687) (end 174.05 60.15) (width 0.25) (layer "B.Cu") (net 1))
 (segment (start 170.053 58.15) (end 174.05 58.15) (width 0.25) (layer "F.Cu") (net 2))
 (segment (start 170.005547 58.102547) (end 170.053 58.15) (width 0.25) (layer "F.Cu") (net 2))
 (via (at 170.005547 58.102547) (size 0.8) (drill 0.4) (layers "F.Cu" "B.Cu") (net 2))
 (segment (start 175.137 60.124251) (end 175.137 59.237) (width 0.25) (layer "B.Cu") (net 2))
 (segment (start 179.2022 60.6252) (end 179.2022 60.8786) (width 0.25) (layer "B.Cu") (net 2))
 (segment (start 169.7642 57.8612) (end 167.5638 57.8612) (width 0.25) (layer "B.Cu") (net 2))
 (segment (start 175.137 59.237) (end 174.05 58.15) (width 0.25) (layer "B.Cu") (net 2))
 (segment (start 178.8438 61.237) (end 176.249749 61.237) (width 0.25) (layer "B.Cu") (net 2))
 (segment (start 173.7612 57.8612) (end 174.05 58.15) (width 0.25) (layer "B.Cu") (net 2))
 (segment (start 173.8816 58.3184) (end 174.05 58.15) (width 0.25) (layer "B.Cu") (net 2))
 (segment (start 179.2022 60.8786) (end 178.8438 61.237) (width 0.25) (layer "B.Cu") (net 2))
 (segment (start 170.005547 58.102547) (end 169.7642 57.8612) (width 0.25) (layer "B.Cu") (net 2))
 (segment (start 176.249749 61.237) (end 175.137 60.124251) (width 0.25) (layer "B.Cu") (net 2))
 (segment (start 177.164928 54.15) (end 177.648964 54.634036) (width 0.25) (layer "F.Cu") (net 5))
 (segment (start 177.556327 54.5414) (end 180.094393 57.079466) (width 0.25) (layer "F.Cu") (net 5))
 (segment (start 176.7 54.15) (end 177.164928 54.15) (width 0.25) (layer "F.Cu") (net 5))
 (via (at 180.094393 57.079466) (size 0.8) (drill 0.4) (layers "F.Cu" "B.Cu") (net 5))
 (segment (start 179.8522 56.837273) (end 179.8522 55.9666) (width 0.25) (layer "B.Cu") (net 5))
 (segment (start 180.094393 57.079466) (end 179.8522 56.837273) (width 0.25) (layer "B.Cu") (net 5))
 (segment (start 182.1896 57.0634) (end 183.1848 57.0634) (width 0.25) (layer "B.Cu") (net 5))
 (segment (start 180.094393 57.079466) (end 182.173534 57.079466) (width 0.25) (layer "B.Cu") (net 5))
 (segment (start 182.173534 57.079466) (end 182.1896 57.0634) (width 0.25) (layer "B.Cu") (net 5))
 (segment (start 182.8038 59.1624) (end 181.513 57.8716) (width 0.25) (layer "B.Cu") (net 6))
 (segment (start 177.3182 56.7682) (end 177.853399 57.303399) (width 0.25) (layer "B.Cu") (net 6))
 (segment (start 179.233602 57.8716) (end 178.665401 57.303399) (width 0.25) (layer "B.Cu") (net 6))
 (segment (start 177.853399 57.303399) (end 178.665401 57.303399) (width 0.25) (layer "B.Cu") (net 6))
 (segment (start 176.7 56.15) (end 177.461999 56.911999) (width 0.25) (layer "B.Cu") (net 6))
 (segment (start 178.665401 57.303399) (end 179.2022 56.7666) (width 0.25) (layer "B.Cu") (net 6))
 (segment (start 181.513 57.8716) (end 179.233602 57.8716) (width 0.25) (layer "B.Cu") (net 6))
 (segment (start 179.2022 56.7666) (end 179.2022 55.9666) (width 0.25) (layer "B.Cu") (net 6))
 (segment (start 178.5522 55.9666) (end 178.5522 55.017) (width 0.25) (layer "B.Cu") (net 10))
 (segment (start 178.5874 55.9314) (end 178.5522 55.9666) (width 0.25) (layer "B.Cu") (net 10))
 (segment (start 178.5522 55.017) (end 178.2064 54.6712) (width 0.25) (layer "B.Cu") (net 10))
 (segment (start 171.3718 57.2008) (end 171.3718 57.7616) (width 0.25) (layer "B.Cu") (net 7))
 (segment (start 171.3718 57.7616) (end 169.2448 59.8886) (width 0.25) (layer "B.Cu") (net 7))
 (segment (start 169.2448 59.8886) (end 167.5638 59.8886) (width 0.25) (layer "B.Cu") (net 7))
 (segment (start 167.8732 56.8706) (end 167.5638 56.5612) (width 0.25) (layer "B.Cu") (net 8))
 (segment (start 171.3738 56.1848) (end 167.9402 56.1848) (width 0.25) (layer "B.Cu") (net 8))
 (segment (start 167.9402 56.1848) (end 167.5638 56.5612) (width 0.25) (layer "B.Cu") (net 8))
 (segment (start 181.229 53.6512) (end 183.1848 55.607) (width 0.25) (layer "B.Cu") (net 9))
 (segment (start 182.6768 54.073694) (end 182.6768 59.8574) (width 0.25) (layer "F.Cu") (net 11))
 (segment (start 182.6768 59.8574) (end 183.261 60.4416) (width 0.25) (layer "F.Cu") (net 11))
 (segment (start 182.157553 53.554447) (end 182.6768 54.073694) (width 0.25) (layer "F.Cu") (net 11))
 (via (at 183.261 60.4416) (size 0.8) (drill 0.4) (layers "F.Cu" "B.Cu") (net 11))
 (via (at 182.157553 53.554447) (size 0.8) (drill 0.4) (layers "F.Cu" "B.Cu") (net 11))
 (segment (start 180.8164 53.0562) (end 180.812 53.0606) (width 0.25) (layer "B.Cu") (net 11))
 (segment (start 181.659306 53.0606) (end 181.654906 53.0562) (width 0.25) (layer "B.Cu") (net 11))
 (segment (start 182.157553 53.554447) (end 181.659306 53.0562) (width 0.25) (layer "B.Cu") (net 11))
 (segment (start 181.654906 53.0562) (end 180.8164 53.0562) (width 0.25) (layer "B.Cu") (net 11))
 (segment (start 180.812 53.0562) (end 180.213 53.6552) (width 0.25) (layer "B.Cu") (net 11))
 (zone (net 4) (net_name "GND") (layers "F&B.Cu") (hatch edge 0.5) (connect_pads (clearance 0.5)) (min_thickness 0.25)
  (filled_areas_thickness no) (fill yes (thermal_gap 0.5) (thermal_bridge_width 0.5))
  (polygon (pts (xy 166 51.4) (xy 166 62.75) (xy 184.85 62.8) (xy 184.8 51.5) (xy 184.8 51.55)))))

